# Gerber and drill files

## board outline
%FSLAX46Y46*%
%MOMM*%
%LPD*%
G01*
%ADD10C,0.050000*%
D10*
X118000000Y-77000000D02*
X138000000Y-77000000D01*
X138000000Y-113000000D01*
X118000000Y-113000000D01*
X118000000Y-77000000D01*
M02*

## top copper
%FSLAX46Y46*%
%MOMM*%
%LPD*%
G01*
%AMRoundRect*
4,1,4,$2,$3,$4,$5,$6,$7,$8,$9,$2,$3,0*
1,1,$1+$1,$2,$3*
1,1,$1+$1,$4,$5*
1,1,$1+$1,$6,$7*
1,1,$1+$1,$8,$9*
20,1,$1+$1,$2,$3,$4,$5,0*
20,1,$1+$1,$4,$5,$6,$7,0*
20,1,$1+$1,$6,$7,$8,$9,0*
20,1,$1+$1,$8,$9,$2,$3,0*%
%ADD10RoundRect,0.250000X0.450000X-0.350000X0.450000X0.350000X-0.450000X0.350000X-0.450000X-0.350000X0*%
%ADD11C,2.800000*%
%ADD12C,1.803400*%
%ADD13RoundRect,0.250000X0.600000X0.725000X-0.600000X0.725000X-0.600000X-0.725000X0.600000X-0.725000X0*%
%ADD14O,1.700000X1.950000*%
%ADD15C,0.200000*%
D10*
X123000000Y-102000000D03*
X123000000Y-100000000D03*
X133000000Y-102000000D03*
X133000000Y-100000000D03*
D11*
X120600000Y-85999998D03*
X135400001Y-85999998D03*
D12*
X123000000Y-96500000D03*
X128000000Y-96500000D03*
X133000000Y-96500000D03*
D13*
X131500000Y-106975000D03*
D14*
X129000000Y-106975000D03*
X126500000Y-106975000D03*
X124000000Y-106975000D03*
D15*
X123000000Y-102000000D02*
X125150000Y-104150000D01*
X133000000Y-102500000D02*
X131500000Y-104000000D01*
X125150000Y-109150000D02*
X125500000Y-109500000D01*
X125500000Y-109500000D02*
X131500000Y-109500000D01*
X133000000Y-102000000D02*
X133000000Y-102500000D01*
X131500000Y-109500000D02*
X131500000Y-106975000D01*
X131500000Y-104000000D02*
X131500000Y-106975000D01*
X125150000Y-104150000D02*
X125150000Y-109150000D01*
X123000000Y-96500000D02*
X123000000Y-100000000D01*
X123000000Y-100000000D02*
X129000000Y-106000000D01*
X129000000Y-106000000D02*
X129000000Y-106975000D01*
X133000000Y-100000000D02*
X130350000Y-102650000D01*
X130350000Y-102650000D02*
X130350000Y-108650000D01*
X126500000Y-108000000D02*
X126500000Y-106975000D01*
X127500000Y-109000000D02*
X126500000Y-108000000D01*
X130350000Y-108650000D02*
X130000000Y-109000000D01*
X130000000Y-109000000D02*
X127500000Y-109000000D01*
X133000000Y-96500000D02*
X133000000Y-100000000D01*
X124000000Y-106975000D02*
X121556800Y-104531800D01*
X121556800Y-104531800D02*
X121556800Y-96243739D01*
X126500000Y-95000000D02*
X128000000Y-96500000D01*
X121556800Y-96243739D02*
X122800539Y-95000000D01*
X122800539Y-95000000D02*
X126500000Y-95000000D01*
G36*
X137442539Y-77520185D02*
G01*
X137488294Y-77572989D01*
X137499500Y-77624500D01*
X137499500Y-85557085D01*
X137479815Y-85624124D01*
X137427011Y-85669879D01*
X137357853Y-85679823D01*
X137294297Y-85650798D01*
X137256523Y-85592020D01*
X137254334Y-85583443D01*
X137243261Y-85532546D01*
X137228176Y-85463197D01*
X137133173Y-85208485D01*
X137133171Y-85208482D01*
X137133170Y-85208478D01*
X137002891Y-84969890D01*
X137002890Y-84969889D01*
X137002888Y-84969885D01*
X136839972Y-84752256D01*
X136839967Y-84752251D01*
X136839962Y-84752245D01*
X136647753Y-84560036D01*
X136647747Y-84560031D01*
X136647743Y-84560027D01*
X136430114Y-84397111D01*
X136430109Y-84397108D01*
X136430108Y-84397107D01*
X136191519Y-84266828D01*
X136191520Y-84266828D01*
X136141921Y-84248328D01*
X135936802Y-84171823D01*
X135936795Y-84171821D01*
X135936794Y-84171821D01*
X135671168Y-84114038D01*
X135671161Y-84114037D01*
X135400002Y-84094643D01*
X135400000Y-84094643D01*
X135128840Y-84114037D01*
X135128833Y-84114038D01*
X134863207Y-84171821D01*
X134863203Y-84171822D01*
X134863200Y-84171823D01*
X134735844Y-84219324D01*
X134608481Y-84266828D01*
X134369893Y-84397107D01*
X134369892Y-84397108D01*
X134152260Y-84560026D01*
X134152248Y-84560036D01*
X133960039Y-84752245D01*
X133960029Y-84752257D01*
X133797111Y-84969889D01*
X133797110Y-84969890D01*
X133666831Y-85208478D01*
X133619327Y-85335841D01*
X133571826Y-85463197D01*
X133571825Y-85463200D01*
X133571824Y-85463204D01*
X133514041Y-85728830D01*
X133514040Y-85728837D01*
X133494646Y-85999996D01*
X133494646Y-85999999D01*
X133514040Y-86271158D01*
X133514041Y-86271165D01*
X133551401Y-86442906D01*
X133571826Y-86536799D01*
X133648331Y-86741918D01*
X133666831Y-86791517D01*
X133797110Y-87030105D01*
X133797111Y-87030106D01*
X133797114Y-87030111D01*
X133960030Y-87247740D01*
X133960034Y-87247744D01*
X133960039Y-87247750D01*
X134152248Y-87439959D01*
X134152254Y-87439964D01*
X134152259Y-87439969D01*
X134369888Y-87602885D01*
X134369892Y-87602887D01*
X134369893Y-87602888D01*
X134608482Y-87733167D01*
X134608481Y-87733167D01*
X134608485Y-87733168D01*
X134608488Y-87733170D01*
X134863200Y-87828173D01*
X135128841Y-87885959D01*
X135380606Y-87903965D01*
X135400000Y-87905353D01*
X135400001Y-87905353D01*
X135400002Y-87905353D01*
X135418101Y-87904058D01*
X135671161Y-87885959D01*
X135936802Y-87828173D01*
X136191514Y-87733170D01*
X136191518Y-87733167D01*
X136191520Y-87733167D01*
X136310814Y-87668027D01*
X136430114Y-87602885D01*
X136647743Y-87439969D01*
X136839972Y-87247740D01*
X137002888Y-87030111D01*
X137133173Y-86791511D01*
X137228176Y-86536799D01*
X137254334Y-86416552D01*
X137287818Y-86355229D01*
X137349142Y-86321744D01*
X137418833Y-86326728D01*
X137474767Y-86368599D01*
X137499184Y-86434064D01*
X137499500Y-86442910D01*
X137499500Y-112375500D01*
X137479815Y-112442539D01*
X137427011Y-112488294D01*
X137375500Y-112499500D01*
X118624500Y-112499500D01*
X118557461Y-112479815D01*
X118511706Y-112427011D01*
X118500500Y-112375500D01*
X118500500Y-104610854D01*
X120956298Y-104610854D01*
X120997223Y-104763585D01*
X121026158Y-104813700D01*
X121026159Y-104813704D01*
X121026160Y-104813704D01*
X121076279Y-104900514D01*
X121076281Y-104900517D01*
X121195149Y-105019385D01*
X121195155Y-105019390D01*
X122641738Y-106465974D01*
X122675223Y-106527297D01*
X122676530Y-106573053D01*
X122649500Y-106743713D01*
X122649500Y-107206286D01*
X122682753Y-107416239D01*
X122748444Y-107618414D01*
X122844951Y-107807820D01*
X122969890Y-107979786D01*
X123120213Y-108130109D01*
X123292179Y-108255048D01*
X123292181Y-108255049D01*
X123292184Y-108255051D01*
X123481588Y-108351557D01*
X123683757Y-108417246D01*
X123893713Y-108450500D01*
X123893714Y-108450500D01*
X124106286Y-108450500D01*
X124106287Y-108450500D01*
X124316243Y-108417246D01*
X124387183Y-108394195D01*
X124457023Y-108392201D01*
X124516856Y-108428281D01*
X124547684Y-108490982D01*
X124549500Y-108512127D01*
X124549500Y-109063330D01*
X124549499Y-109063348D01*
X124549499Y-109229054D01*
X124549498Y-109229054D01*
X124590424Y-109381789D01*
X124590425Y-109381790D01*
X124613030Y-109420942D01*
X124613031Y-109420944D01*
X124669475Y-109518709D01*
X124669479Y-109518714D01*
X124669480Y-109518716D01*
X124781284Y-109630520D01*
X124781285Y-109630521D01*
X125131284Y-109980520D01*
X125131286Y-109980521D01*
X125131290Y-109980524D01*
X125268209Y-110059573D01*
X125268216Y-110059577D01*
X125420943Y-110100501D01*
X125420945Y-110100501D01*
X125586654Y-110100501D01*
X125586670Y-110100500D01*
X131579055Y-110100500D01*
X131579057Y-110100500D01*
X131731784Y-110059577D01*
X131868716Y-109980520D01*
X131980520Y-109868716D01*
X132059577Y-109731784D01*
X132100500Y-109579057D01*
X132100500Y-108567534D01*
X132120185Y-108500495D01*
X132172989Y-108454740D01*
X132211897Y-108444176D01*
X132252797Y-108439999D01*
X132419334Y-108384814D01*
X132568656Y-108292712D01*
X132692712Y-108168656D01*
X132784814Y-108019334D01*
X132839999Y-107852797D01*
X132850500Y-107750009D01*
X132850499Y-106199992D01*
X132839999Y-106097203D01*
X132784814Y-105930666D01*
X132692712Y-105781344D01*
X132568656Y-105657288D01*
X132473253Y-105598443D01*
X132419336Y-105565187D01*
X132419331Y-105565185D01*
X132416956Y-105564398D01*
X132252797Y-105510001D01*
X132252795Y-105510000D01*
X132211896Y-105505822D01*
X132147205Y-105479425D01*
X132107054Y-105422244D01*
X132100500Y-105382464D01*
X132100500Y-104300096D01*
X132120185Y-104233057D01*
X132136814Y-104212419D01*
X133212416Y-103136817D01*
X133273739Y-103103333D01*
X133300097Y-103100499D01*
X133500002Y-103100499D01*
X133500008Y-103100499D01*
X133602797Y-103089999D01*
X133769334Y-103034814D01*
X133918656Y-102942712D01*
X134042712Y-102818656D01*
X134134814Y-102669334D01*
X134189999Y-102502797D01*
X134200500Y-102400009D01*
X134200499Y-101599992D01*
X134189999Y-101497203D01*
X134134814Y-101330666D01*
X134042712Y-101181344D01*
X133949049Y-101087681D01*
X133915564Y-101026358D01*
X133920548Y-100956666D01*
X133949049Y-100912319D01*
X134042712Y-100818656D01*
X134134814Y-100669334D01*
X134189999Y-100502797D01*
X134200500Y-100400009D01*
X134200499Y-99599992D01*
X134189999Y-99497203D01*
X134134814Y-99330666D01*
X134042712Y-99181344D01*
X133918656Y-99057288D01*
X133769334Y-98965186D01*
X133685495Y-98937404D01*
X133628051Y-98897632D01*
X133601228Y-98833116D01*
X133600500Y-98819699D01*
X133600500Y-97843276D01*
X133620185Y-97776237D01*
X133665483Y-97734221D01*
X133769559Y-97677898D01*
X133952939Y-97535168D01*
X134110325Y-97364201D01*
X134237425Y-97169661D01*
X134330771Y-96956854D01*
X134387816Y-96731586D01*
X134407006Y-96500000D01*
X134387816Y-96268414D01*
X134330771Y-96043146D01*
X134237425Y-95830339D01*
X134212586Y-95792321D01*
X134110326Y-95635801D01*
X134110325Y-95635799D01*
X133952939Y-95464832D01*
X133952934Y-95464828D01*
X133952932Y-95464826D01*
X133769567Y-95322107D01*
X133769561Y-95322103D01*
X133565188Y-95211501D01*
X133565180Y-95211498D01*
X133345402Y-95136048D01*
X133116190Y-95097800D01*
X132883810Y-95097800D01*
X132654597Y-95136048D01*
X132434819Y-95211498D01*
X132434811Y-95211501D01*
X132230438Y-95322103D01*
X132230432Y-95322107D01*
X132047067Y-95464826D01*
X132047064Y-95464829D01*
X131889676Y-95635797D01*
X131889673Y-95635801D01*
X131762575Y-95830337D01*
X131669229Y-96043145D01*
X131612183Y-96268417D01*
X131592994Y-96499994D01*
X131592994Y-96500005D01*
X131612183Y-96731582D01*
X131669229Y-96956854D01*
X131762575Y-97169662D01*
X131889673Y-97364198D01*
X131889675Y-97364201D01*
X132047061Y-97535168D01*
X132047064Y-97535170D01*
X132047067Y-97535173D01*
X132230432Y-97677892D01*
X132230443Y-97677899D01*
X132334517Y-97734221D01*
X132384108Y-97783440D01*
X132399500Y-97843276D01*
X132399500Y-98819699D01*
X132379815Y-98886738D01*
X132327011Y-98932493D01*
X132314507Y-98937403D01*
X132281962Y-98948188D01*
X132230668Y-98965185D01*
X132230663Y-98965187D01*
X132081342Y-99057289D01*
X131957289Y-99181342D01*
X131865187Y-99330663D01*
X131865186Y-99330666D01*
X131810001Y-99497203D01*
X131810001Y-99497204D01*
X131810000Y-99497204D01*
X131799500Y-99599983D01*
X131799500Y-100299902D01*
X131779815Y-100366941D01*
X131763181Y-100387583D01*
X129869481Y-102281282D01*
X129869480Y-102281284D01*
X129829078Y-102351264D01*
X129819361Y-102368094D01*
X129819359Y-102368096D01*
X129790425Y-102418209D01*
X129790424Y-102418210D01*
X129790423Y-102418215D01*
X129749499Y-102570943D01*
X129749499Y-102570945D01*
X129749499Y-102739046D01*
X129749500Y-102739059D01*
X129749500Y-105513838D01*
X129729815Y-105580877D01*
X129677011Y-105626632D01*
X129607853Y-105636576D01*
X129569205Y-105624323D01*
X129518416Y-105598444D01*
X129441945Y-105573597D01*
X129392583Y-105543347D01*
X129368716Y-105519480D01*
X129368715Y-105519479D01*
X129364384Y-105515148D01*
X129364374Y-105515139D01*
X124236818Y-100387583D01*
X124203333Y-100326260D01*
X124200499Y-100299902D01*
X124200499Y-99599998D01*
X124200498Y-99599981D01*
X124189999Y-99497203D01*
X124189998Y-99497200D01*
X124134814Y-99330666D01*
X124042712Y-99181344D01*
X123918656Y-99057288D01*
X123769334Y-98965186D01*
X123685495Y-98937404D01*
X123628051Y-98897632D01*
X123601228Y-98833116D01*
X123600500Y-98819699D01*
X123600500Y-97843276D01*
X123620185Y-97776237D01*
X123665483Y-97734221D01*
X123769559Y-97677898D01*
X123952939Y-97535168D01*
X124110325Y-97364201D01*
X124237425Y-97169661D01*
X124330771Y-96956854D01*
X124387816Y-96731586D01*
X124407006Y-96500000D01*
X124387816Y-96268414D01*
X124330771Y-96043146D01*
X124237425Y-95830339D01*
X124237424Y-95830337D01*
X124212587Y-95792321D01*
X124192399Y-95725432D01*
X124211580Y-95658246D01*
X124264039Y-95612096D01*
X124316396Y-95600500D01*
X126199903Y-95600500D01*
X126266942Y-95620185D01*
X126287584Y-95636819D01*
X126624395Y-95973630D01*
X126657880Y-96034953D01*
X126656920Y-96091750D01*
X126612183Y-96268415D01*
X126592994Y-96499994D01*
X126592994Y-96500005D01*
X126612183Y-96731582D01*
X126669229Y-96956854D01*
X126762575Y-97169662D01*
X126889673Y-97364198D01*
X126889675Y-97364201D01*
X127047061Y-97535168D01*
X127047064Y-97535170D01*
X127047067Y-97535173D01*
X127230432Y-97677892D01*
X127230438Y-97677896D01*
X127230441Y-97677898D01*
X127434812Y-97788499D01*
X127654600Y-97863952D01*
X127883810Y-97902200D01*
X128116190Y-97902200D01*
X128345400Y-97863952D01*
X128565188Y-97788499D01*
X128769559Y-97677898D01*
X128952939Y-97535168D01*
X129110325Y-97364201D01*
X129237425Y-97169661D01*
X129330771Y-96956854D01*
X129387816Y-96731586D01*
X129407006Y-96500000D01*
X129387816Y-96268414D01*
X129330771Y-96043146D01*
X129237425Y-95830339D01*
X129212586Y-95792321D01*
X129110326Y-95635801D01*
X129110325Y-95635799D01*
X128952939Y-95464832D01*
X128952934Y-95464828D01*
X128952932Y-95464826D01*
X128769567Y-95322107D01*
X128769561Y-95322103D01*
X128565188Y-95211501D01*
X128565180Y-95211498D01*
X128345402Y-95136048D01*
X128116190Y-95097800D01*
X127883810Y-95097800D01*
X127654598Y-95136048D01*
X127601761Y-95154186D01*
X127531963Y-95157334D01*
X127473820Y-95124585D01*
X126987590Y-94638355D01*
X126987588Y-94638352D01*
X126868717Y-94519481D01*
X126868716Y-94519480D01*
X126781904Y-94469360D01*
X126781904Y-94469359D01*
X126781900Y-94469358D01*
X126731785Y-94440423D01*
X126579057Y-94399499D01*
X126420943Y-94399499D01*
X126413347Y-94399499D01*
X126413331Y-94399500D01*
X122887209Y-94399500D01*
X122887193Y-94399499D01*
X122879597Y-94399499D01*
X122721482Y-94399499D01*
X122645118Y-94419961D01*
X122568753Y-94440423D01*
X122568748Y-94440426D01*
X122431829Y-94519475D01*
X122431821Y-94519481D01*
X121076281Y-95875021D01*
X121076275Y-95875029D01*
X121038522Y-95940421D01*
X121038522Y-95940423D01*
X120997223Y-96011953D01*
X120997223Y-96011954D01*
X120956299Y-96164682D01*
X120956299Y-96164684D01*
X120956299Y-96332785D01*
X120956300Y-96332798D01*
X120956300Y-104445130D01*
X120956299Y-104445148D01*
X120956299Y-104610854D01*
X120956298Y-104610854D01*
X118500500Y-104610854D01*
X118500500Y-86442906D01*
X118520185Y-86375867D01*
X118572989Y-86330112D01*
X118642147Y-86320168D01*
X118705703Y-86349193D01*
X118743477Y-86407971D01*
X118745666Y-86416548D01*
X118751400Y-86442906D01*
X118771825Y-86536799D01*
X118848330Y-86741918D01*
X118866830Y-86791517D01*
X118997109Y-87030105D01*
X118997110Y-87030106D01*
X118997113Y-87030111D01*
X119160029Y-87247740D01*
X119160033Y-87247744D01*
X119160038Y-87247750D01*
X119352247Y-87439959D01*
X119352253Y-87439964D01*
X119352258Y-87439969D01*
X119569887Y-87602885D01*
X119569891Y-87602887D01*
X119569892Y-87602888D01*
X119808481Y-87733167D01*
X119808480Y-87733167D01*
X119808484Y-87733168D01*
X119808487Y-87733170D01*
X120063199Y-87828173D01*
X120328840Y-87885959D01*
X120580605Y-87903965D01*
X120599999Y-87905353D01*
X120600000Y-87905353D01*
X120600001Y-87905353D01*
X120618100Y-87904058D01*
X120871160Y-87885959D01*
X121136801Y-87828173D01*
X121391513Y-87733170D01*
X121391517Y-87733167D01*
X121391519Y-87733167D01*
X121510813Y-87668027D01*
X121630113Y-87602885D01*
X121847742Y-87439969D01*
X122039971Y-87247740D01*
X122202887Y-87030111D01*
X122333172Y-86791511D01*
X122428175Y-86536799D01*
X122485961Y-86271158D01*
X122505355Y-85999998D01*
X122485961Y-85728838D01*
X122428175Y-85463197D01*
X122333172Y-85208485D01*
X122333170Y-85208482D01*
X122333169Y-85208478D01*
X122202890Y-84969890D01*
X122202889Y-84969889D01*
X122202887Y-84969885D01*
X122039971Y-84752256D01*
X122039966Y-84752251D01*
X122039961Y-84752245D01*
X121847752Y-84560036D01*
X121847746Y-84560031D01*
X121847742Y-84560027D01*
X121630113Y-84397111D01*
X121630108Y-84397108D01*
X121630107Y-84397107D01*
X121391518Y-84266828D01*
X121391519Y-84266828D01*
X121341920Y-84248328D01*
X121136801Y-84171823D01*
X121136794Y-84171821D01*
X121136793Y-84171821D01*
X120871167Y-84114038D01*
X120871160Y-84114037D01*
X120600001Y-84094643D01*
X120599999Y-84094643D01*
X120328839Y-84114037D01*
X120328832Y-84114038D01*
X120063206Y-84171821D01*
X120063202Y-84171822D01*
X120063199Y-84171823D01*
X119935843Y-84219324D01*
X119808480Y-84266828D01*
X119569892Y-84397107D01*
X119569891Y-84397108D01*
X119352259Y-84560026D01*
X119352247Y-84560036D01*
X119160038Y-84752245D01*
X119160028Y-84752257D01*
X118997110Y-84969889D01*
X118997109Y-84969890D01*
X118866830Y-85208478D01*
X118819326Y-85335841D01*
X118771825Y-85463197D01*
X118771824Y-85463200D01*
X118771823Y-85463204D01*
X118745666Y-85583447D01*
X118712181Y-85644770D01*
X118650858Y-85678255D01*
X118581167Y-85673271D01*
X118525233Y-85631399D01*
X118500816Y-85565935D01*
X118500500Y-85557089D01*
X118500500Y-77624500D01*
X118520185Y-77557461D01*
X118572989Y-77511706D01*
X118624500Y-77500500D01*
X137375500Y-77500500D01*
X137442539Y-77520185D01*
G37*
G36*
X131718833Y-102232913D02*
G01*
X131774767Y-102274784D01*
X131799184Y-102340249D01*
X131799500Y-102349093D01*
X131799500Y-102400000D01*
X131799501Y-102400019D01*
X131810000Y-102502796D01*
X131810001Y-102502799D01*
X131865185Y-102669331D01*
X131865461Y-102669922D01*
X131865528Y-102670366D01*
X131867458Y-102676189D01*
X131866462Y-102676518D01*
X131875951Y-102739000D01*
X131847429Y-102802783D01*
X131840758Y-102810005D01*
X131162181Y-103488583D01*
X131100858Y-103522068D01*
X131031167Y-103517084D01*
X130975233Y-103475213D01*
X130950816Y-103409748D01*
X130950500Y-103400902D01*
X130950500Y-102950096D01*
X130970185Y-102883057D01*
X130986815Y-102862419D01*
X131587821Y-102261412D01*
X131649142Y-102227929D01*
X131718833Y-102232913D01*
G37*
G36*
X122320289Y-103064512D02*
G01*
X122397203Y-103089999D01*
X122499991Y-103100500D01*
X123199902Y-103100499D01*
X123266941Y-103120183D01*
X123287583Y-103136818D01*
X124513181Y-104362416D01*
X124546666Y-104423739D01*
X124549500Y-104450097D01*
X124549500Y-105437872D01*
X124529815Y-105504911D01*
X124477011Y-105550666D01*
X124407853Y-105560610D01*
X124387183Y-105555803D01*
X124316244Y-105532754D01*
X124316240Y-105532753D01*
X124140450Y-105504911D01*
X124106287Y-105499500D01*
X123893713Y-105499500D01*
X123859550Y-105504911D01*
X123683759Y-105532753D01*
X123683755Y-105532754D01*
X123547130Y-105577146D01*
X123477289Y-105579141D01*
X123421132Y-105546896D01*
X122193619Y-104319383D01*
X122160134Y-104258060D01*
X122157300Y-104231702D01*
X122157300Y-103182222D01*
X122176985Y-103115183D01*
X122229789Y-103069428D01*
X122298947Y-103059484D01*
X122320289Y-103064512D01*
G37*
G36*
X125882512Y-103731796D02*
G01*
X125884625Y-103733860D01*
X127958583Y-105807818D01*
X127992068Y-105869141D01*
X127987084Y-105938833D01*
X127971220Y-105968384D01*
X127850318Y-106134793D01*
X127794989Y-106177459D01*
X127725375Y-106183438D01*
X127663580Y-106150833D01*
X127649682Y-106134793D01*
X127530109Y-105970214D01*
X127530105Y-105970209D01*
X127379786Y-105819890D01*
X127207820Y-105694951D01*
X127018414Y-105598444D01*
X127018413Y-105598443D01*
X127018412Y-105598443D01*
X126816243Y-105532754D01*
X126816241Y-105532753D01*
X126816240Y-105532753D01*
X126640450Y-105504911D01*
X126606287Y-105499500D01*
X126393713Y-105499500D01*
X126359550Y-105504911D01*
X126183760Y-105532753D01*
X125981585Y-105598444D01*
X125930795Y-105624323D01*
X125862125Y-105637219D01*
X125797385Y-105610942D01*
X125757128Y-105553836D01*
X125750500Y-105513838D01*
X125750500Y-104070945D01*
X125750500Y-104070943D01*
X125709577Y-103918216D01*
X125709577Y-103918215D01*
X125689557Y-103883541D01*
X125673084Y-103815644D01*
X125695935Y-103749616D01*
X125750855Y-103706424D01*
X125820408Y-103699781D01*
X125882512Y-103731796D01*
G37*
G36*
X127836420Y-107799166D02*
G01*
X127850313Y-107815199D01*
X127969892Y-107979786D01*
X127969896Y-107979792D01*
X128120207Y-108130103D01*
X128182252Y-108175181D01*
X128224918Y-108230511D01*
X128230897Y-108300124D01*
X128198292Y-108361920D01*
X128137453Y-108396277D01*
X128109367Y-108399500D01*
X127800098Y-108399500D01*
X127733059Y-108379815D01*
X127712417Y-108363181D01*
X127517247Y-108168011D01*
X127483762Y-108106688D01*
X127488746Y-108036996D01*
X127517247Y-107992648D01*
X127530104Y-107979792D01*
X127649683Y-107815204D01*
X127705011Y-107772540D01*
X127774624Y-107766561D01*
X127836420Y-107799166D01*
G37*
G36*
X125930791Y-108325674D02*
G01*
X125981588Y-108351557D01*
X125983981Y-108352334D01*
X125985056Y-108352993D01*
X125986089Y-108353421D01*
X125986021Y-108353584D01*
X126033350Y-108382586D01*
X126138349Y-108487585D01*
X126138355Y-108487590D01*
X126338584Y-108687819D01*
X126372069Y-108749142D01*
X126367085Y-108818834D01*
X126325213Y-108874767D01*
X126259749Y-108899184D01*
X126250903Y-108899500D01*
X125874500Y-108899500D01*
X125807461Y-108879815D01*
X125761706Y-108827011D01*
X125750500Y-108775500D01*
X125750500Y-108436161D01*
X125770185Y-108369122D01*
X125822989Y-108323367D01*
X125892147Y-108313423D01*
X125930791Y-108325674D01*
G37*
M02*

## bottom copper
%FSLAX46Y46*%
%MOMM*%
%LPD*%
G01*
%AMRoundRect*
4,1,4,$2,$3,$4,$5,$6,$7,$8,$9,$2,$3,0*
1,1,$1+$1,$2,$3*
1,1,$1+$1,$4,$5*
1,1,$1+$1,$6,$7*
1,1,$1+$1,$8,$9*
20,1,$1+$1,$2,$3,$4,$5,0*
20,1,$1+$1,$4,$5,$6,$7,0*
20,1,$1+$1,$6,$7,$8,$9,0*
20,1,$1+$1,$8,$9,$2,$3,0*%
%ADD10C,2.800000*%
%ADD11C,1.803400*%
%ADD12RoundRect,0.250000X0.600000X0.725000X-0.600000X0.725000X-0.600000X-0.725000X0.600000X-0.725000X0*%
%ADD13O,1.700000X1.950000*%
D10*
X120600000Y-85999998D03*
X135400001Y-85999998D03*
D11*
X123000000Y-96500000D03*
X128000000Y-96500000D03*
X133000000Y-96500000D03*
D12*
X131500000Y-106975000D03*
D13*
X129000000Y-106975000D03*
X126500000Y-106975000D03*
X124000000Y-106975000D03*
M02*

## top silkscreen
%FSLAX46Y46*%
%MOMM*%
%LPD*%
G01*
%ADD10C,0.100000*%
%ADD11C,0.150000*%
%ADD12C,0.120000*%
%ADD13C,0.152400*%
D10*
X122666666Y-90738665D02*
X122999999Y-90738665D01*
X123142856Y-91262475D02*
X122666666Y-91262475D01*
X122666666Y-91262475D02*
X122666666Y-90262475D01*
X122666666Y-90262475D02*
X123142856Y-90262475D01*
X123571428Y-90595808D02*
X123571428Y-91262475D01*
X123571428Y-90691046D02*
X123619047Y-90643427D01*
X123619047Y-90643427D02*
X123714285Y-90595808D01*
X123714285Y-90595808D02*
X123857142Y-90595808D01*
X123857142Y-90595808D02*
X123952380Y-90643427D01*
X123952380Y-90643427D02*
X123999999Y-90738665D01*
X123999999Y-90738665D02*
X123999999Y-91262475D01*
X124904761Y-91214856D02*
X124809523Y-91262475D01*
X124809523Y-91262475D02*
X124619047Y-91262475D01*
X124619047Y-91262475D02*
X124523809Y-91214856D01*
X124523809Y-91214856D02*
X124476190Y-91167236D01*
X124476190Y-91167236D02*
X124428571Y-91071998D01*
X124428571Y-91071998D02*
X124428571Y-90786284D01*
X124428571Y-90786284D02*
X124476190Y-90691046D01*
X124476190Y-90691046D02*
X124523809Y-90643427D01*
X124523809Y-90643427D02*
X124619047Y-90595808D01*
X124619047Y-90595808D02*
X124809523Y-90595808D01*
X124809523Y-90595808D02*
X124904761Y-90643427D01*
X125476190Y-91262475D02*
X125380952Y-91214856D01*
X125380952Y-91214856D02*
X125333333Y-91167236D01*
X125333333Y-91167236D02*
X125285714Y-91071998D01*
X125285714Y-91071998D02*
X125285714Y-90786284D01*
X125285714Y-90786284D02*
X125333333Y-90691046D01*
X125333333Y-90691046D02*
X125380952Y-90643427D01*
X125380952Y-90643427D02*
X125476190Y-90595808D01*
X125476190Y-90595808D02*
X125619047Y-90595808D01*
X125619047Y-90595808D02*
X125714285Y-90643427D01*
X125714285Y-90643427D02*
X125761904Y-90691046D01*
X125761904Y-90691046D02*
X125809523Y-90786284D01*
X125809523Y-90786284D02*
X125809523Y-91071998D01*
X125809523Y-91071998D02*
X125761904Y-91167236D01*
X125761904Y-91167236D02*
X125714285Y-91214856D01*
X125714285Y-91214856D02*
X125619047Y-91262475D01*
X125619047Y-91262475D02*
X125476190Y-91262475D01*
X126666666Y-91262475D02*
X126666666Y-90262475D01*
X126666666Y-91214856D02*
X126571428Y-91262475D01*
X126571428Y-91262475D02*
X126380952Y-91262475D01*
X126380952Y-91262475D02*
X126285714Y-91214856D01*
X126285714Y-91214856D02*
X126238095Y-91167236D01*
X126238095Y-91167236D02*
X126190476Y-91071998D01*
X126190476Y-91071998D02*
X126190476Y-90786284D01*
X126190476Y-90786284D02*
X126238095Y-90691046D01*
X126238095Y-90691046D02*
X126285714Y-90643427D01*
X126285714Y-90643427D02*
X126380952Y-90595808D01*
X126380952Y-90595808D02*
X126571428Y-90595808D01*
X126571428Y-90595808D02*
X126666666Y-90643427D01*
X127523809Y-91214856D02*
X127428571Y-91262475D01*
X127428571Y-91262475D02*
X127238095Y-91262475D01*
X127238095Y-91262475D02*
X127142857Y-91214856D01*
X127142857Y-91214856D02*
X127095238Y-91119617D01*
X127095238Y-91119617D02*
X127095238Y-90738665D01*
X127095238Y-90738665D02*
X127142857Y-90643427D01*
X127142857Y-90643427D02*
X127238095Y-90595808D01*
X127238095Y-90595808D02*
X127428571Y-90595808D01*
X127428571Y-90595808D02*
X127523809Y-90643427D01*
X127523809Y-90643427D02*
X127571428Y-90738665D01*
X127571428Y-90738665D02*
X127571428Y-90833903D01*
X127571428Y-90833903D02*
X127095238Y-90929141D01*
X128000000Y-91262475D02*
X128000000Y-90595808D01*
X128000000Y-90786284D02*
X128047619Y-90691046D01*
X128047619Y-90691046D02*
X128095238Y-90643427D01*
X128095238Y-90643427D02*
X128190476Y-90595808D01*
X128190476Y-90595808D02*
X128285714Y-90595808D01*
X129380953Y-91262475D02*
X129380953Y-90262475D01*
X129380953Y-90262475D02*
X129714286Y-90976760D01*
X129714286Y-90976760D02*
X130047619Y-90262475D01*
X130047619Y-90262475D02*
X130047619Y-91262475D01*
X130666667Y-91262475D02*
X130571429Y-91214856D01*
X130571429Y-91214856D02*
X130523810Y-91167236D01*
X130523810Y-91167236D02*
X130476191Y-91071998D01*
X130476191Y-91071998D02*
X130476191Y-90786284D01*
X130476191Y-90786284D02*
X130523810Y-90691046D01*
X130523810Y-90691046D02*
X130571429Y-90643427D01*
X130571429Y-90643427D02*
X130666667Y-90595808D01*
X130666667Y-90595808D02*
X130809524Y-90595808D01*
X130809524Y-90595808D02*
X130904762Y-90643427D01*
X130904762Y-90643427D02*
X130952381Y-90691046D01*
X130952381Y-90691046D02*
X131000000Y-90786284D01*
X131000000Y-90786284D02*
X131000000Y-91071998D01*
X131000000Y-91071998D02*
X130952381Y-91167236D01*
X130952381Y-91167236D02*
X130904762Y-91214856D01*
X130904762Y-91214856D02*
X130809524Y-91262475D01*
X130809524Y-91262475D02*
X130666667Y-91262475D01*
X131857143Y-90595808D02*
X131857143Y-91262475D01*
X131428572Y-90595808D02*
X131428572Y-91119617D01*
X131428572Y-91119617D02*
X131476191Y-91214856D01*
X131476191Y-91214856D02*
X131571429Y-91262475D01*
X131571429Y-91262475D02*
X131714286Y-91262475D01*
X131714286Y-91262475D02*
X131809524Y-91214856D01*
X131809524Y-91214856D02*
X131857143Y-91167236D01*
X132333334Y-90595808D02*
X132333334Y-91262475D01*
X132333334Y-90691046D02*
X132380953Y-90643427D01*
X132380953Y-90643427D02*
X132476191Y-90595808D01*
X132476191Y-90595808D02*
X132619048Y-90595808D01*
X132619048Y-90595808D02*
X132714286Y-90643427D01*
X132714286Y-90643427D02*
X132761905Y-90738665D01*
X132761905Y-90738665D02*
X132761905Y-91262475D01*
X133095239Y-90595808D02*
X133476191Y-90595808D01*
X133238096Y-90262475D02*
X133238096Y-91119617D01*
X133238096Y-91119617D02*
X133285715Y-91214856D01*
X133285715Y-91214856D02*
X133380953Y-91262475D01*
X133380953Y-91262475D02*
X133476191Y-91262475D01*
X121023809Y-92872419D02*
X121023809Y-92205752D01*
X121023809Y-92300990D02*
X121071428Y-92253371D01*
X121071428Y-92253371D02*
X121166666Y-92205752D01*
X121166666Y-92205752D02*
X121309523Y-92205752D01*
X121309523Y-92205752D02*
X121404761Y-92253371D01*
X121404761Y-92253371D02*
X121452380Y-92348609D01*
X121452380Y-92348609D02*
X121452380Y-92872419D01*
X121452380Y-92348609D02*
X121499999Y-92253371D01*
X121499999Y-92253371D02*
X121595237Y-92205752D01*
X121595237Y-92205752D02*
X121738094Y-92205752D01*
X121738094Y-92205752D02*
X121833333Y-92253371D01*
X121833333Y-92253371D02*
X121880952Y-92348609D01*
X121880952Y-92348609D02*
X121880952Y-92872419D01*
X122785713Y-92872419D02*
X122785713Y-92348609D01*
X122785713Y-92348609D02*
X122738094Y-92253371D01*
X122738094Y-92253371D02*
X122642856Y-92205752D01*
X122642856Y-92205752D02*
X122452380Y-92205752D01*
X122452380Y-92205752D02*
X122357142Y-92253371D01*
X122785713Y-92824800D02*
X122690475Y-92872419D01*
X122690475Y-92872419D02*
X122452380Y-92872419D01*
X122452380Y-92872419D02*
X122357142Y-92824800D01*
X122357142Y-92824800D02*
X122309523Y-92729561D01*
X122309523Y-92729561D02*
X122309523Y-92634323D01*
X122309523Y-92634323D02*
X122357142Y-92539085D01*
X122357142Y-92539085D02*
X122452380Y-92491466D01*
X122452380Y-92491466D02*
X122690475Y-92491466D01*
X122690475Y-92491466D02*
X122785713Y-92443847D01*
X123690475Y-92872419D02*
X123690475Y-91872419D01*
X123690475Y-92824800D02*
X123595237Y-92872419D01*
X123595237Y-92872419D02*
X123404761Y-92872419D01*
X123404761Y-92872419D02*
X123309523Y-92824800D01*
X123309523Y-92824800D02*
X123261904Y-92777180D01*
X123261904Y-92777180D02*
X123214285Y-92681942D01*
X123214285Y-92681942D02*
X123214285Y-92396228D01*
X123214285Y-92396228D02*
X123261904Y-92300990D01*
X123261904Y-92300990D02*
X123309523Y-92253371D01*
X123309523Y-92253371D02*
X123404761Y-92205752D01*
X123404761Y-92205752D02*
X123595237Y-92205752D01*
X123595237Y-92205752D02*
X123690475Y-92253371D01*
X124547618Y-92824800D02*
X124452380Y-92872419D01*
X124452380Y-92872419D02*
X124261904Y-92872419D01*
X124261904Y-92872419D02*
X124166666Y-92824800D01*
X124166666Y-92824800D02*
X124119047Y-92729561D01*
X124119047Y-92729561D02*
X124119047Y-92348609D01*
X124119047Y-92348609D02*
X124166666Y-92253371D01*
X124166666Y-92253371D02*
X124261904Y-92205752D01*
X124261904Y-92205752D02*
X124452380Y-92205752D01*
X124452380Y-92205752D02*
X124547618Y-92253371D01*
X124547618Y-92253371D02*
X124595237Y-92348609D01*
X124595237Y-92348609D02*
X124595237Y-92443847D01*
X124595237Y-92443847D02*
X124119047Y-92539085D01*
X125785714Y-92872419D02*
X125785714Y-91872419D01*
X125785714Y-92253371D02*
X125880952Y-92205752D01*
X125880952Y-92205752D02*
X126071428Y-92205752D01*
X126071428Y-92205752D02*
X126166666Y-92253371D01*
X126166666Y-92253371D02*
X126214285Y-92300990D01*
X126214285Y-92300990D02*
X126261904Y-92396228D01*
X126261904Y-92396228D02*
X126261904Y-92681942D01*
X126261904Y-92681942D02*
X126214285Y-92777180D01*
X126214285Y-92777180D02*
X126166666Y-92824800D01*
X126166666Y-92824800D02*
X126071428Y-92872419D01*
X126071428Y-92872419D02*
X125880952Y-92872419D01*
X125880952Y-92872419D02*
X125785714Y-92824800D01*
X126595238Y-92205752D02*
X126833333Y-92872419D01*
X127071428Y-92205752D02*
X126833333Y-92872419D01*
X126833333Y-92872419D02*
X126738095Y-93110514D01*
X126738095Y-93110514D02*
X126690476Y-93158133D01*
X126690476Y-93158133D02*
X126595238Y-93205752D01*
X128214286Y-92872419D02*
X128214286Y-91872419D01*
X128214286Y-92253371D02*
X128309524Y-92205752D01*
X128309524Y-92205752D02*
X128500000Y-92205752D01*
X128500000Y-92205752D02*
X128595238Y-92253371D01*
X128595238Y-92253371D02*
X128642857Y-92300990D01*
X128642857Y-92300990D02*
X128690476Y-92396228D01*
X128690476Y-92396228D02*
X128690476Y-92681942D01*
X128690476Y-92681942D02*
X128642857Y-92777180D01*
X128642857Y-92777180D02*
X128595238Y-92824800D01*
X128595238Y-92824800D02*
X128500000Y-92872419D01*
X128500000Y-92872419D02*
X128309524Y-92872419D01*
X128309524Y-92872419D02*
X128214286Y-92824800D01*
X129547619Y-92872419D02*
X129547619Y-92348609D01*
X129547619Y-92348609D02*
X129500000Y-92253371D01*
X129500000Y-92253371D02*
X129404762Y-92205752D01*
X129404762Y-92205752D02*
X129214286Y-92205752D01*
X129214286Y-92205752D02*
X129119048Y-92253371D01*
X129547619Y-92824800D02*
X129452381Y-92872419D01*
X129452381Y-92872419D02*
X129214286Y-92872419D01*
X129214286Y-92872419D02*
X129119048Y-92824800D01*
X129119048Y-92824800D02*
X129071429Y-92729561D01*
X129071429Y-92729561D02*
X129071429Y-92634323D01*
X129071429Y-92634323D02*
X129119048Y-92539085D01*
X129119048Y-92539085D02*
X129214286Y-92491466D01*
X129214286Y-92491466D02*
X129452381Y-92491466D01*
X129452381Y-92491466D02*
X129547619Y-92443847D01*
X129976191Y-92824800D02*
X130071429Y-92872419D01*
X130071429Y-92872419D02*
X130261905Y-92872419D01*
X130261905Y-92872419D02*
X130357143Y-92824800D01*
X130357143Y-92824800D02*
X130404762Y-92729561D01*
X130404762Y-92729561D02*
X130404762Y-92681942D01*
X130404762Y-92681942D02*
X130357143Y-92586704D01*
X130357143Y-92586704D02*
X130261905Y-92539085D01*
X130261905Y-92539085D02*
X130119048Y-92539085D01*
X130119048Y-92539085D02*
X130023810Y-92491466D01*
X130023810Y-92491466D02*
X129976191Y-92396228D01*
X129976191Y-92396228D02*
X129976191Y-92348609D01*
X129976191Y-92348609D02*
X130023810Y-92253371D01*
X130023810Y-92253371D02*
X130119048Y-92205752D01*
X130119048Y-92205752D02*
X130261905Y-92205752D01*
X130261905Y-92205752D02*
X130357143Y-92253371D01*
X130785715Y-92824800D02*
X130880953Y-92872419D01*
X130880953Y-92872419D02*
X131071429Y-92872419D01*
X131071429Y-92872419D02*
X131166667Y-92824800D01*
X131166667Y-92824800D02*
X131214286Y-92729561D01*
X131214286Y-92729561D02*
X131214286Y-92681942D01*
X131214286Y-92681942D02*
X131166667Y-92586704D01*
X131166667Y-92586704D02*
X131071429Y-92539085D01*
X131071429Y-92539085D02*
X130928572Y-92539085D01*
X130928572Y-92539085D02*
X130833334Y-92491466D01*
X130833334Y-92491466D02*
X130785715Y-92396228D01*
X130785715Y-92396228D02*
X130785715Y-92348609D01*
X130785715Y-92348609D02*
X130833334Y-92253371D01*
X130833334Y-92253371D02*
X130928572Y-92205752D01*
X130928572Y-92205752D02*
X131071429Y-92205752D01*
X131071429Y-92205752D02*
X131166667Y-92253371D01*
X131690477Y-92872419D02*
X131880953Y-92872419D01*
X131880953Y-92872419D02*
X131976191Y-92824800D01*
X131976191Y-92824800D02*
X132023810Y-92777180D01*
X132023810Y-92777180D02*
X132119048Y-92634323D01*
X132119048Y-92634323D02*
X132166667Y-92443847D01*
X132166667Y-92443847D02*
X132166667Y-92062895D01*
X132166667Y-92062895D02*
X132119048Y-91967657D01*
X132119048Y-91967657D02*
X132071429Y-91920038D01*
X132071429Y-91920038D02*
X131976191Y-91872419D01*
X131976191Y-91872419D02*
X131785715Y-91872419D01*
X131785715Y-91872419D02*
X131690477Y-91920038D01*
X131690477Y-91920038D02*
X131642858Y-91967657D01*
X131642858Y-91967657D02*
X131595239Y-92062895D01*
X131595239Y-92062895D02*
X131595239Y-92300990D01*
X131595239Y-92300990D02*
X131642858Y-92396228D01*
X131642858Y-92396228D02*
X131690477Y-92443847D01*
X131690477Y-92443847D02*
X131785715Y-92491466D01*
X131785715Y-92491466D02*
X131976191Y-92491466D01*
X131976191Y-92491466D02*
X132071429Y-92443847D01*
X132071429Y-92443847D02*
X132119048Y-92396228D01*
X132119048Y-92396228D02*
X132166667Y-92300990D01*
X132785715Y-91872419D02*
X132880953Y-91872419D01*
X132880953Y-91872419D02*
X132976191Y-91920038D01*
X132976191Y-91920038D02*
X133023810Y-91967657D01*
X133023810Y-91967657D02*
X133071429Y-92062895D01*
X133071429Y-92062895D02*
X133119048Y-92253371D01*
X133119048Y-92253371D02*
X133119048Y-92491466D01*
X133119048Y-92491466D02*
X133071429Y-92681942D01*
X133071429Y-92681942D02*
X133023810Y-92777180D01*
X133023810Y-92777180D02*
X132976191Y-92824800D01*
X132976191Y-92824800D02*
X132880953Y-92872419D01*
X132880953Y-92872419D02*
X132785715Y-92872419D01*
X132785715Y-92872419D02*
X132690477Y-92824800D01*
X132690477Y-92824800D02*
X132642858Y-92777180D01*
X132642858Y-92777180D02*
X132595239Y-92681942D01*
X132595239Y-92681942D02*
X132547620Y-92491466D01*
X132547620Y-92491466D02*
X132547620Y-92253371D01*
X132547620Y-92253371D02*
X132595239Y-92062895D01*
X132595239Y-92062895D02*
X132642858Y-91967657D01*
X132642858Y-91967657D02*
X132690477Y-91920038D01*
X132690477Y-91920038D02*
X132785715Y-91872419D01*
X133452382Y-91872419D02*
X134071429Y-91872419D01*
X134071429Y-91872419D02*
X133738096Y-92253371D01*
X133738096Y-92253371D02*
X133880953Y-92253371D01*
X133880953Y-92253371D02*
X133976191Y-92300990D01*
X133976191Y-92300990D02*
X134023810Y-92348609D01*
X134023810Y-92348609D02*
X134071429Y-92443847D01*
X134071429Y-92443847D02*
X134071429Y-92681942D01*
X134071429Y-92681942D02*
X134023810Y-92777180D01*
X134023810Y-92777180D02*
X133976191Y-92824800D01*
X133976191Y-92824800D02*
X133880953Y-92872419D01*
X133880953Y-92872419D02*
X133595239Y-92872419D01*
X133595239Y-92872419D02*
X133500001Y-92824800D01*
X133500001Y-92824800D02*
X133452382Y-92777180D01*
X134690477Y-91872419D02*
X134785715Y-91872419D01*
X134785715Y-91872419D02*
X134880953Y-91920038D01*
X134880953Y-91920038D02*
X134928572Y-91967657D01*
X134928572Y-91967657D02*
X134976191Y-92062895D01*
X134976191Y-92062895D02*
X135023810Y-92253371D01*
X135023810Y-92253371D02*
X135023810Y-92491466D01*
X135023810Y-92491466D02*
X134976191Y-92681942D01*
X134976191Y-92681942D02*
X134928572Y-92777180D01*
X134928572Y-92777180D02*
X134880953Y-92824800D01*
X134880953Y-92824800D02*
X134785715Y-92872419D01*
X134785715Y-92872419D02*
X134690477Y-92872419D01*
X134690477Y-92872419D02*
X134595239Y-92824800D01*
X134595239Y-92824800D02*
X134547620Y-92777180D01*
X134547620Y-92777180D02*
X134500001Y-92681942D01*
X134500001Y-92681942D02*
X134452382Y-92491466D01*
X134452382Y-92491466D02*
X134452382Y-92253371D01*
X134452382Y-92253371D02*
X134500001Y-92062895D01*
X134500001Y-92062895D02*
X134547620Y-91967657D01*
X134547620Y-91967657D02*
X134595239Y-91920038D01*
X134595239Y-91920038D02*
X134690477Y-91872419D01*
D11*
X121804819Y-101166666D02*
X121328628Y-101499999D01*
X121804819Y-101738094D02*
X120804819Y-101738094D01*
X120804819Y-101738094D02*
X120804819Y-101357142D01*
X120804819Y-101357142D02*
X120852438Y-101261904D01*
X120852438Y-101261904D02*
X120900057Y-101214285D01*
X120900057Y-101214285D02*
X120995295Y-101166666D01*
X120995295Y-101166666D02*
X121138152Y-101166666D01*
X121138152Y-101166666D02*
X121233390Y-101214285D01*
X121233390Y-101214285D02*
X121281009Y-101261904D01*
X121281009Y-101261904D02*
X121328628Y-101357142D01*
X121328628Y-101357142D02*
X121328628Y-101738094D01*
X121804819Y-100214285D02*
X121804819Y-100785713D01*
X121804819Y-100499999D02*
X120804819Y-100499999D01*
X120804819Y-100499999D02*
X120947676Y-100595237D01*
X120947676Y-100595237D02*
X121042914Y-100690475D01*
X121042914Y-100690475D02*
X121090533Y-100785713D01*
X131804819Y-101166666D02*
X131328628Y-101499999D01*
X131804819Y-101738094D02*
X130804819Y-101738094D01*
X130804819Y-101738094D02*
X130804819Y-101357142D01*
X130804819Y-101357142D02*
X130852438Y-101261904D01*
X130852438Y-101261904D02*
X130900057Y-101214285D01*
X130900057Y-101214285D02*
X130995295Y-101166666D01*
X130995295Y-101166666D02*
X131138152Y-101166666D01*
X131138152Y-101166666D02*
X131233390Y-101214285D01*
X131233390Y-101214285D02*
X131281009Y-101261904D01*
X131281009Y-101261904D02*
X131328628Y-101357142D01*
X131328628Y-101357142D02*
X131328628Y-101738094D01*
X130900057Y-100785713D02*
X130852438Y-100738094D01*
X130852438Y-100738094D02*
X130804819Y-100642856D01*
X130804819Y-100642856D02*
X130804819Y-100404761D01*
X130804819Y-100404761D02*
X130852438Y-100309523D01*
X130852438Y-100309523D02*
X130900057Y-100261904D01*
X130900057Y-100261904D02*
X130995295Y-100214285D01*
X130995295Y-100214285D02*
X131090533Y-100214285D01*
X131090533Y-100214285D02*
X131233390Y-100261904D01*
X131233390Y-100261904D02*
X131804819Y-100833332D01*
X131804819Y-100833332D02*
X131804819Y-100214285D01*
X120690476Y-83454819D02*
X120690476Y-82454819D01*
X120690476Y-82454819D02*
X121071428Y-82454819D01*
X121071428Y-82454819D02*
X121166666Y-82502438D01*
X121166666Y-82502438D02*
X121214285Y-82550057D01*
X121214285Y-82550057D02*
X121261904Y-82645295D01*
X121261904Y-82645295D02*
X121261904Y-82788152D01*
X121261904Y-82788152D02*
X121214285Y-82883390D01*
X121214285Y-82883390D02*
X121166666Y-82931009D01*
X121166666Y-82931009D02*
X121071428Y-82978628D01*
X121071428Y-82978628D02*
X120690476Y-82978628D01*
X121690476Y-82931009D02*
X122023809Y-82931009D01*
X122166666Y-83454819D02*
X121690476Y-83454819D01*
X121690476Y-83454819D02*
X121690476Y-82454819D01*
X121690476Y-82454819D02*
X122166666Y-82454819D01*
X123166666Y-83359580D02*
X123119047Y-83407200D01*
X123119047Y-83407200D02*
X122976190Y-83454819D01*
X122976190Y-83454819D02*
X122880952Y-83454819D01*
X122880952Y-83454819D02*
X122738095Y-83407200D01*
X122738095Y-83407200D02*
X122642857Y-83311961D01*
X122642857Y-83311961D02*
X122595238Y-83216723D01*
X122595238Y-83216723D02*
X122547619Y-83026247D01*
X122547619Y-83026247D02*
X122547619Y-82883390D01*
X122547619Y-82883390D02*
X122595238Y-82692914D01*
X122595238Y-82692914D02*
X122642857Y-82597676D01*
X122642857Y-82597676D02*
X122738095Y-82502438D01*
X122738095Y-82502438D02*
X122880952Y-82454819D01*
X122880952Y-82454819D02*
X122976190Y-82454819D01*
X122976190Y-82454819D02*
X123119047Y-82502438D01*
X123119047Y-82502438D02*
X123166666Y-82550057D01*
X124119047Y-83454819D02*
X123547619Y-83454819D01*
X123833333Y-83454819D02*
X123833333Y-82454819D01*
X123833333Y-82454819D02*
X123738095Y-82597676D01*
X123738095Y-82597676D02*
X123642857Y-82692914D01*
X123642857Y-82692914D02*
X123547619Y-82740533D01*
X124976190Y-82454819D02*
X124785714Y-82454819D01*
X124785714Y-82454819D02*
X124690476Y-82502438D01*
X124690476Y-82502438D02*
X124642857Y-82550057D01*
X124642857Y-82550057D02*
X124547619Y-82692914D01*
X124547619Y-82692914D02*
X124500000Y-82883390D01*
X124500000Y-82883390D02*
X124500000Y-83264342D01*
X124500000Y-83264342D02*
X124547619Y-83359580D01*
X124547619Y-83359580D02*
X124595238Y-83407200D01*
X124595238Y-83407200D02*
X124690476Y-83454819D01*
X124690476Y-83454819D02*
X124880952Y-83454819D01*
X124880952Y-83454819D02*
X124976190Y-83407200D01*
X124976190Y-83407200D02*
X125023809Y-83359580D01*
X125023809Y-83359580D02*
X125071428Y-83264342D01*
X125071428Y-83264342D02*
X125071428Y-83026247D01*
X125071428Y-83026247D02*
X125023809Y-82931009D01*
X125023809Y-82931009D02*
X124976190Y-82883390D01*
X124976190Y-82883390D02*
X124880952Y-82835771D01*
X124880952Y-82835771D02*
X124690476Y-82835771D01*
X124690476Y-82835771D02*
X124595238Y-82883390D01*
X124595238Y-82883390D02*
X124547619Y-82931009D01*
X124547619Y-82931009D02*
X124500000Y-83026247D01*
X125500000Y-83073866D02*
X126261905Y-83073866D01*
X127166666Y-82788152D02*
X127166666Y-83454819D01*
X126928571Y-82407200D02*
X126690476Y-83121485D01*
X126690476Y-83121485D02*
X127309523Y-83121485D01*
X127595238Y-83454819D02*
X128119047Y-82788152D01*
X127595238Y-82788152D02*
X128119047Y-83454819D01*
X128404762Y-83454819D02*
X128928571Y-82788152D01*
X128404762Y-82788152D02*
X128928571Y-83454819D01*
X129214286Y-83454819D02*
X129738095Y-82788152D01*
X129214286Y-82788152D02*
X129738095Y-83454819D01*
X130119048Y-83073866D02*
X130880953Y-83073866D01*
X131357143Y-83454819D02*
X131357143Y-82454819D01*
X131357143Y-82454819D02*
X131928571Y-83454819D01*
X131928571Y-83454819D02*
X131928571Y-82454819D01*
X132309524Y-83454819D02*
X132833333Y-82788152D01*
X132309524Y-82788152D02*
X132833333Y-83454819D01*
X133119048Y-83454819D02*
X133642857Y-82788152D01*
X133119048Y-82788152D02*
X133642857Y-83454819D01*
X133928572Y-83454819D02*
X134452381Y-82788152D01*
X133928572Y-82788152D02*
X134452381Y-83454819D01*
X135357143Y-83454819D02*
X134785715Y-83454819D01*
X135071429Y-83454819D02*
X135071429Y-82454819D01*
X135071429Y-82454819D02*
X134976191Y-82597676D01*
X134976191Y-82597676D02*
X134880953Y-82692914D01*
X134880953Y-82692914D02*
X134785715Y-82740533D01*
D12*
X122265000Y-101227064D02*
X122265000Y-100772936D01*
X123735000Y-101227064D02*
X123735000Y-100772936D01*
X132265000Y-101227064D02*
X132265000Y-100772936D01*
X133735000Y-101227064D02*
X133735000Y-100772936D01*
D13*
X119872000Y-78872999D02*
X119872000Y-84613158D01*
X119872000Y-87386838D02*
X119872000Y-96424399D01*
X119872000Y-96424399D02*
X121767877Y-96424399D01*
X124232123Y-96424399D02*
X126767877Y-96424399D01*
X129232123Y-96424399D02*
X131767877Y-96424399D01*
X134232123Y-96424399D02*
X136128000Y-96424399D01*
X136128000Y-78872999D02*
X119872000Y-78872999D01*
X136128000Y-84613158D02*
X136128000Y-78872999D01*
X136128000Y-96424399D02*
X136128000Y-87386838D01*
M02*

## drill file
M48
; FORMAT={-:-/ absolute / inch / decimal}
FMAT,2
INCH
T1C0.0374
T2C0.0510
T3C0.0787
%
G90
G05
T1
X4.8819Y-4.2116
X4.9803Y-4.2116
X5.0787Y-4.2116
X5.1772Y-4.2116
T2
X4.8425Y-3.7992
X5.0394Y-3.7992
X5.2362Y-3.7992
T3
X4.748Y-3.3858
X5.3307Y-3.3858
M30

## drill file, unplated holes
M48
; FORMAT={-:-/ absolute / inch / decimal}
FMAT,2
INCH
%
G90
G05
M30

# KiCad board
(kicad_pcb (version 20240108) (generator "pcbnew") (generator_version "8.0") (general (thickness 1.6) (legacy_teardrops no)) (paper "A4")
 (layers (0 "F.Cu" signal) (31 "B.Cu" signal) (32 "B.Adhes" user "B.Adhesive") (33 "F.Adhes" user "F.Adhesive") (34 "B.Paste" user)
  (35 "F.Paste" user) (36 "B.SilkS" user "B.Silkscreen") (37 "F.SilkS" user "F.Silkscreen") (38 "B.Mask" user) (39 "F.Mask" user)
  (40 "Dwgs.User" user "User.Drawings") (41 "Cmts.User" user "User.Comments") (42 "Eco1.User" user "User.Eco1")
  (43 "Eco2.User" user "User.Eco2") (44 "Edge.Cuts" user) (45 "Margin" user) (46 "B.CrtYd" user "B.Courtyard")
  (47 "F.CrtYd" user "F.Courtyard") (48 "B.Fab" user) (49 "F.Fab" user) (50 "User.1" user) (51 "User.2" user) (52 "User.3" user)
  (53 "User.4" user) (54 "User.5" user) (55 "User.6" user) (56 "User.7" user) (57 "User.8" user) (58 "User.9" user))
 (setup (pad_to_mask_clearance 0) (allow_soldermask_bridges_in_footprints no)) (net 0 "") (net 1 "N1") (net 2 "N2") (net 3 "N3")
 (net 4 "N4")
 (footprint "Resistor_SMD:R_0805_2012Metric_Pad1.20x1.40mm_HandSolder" (layer "F.Cu") (at 123 101 90)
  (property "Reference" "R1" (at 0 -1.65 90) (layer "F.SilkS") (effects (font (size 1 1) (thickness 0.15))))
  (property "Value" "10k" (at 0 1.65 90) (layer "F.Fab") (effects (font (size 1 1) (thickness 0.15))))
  (fp_line (start -0.227064 -0.735) (end 0.227064 -0.735) (stroke (width 0.12) (type solid)) (layer "F.SilkS"))
  (fp_line (start -0.227064 0.735) (end 0.227064 0.735) (stroke (width 0.12) (type solid)) (layer "F.SilkS"))
  (pad "1" smd roundrect (at -1 0 90) (size 1.2 1.4) (layers "F.Cu" "F.Paste" "F.Mask") (roundrect_rratio 0.208333) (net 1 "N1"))
  (pad "2" smd roundrect (at 1 0 90) (size 1.2 1.4) (layers "F.Cu" "F.Paste" "F.Mask") (roundrect_rratio 0.208333) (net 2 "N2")))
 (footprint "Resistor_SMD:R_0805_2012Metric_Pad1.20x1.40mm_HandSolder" (layer "F.Cu") (at 133 101 90)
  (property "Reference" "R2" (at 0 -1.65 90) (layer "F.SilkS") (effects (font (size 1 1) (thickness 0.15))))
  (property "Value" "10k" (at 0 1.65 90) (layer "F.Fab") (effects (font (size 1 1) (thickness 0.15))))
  (fp_line (start -0.227064 -0.735) (end 0.227064 -0.735) (stroke (width 0.12) (type solid)) (layer "F.SilkS"))
  (fp_line (start -0.227064 0.735) (end 0.227064 0.735) (stroke (width 0.12) (type solid)) (layer "F.SilkS"))
  (pad "1" smd roundrect (at -1 0 90) (size 1.2 1.4) (layers "F.Cu" "F.Paste" "F.Mask") (roundrect_rratio 0.208333) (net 1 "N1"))
  (pad "2" smd roundrect (at 1 0 90) (size 1.2 1.4) (layers "F.Cu" "F.Paste" "F.Mask") (roundrect_rratio 0.208333) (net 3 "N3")))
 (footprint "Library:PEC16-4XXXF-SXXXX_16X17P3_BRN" (layer "F.Cu") (at 135.400001 85.999998)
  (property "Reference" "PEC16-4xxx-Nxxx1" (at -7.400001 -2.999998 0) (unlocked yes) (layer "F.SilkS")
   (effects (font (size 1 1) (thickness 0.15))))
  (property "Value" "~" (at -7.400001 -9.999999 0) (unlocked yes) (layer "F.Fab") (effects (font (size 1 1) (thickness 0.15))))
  (fp_line (start -15.528001 -7.126999) (end -15.528001 -1.38684) (stroke (width 0.1524) (type solid)) (layer "F.SilkS"))
  (fp_line (start -15.528001 1.38684) (end -15.528001 10.424401) (stroke (width 0.1524) (type solid)) (layer "F.SilkS"))
  (fp_line (start -15.528001 10.424401) (end -13.632124 10.424401) (stroke (width 0.1524) (type solid)) (layer "F.SilkS"))
  (fp_line (start -11.167878 10.424401) (end -8.632124 10.424401) (stroke (width 0.1524) (type solid)) (layer "F.SilkS"))
  (fp_line (start -6.167878 10.424401) (end -3.632124 10.424401) (stroke (width 0.1524) (type solid)) (layer "F.SilkS"))
  (fp_line (start -1.167878 10.424401) (end 0.727999 10.424401) (stroke (width 0.1524) (type solid)) (layer "F.SilkS"))
  (fp_line (start 0.727999 -7.126999) (end -15.528001 -7.126999) (stroke (width 0.1524) (type solid)) (layer "F.SilkS"))
  (fp_line (start 0.727999 -1.38684) (end 0.727999 -7.126999) (stroke (width 0.1524) (type solid)) (layer "F.SilkS"))
  (fp_line (start 0.727999 10.424401) (end 0.727999 1.38684) (stroke (width 0.1524) (type solid)) (layer "F.SilkS"))
  (pad "" thru_hole circle (at -14.800001 0) (size 2.8 2.8) (drill 2) (layers "*.Cu" "*.Mask") (remove_unused_layers no))
  (pad "" thru_hole circle (at 0 0) (size 2.8 2.8) (drill 2) (layers "*.Cu" "*.Mask") (remove_unused_layers no))
  (pad "1" thru_hole circle (at -12.400001 10.500002) (size 1.8034 1.8034) (drill 1.2954) (layers "*.Cu" "*.Mask") (remove_unused_layers no)
   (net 2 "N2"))
  (pad "2" thru_hole circle (at -7.400001 10.500002) (size 1.8034 1.8034) (drill 1.2954) (layers "*.Cu" "*.Mask") (remove_unused_layers no)
   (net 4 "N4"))
  (pad "3" thru_hole circle (at -2.400001 10.500002) (size 1.8034 1.8034) (drill 1.2954) (layers "*.Cu" "*.Mask") (remove_unused_layers no)
   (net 3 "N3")))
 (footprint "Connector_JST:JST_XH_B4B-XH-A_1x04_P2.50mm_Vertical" (layer "B.Cu") (at 131.5 106.975 180)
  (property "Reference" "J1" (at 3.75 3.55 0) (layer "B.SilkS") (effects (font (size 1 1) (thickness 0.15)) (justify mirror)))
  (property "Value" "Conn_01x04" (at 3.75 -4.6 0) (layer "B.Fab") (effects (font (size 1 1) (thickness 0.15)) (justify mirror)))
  (pad "1" thru_hole roundrect (at 0 0 180) (size 1.7 1.95) (drill 0.95) (layers "*.Cu" "*.Mask") (remove_unused_layers no)
   (roundrect_rratio 0.147059) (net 1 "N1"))
  (pad "2" thru_hole oval (at 2.5 0 180) (size 1.7 1.95) (drill 0.95) (layers "*.Cu" "*.Mask") (remove_unused_layers no) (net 2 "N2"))
  (pad "3" thru_hole oval (at 5 0 180) (size 1.7 1.95) (drill 0.95) (layers "*.Cu" "*.Mask") (remove_unused_layers no) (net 3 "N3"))
  (pad "4" thru_hole oval (at 7.5 0 180) (size 1.7 1.95) (drill 0.95) (layers "*.Cu" "*.Mask") (remove_unused_layers no) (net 4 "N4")))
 (gr_rect (start 118 77) (end 138 113) (stroke (width 0.05) (type default)) (fill none) (layer "Edge.Cuts"))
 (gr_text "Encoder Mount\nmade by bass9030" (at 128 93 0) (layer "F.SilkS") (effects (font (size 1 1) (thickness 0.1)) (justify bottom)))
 (segment (start 123 102) (end 125.15 104.15) (width 0.2) (layer "F.Cu") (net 1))
 (segment (start 133 102.5) (end 131.5 104) (width 0.2) (layer "F.Cu") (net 1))
 (segment (start 125.15 109.15) (end 125.5 109.5) (width 0.2) (layer "F.Cu") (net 1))
 (segment (start 125.5 109.5) (end 131.5 109.5) (width 0.2) (layer "F.Cu") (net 1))
 (segment (start 133 102) (end 133 102.5) (width 0.2) (layer "F.Cu") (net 1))
 (segment (start 131.5 109.5) (end 131.5 106.975) (width 0.2) (layer "F.Cu") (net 1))
 (segment (start 131.5 104) (end 131.5 106.975) (width 0.2) (layer "F.Cu") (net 1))
 (segment (start 125.15 104.15) (end 125.15 109.15) (width 0.2) (layer "F.Cu") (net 1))
 (segment (start 123 96.5) (end 123 100) (width 0.2) (layer "F.Cu") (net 2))
 (segment (start 123 100) (end 129 106) (width 0.2) (layer "F.Cu") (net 2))
 (segment (start 129 106) (end 129 106.975) (width 0.2) (layer "F.Cu") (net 2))
 (segment (start 133 100) (end 130.35 102.65) (width 0.2) (layer "F.Cu") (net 3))
 (segment (start 130.35 102.65) (end 130.35 108.65) (width 0.2) (layer "F.Cu") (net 3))
 (segment (start 126.5 108) (end 126.5 106.975) (width 0.2) (layer "F.Cu") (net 3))
 (segment (start 127.5 109) (end 126.5 108) (width 0.2) (layer "F.Cu") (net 3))
 (segment (start 130.35 108.65) (end 130 109) (width 0.2) (layer "F.Cu") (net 3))
 (segment (start 130 109) (end 127.5 109) (width 0.2) (layer "F.Cu") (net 3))
 (segment (start 133 96.5) (end 133 100) (width 0.2) (layer "F.Cu") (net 3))
 (segment (start 124 106.975) (end 121.5568 104.5318) (width 0.2) (layer "F.Cu") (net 4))
 (segment (start 121.5568 104.5318) (end 121.5568 96.243739) (width 0.2) (layer "F.Cu") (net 4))
 (segment (start 126.5 95) (end 128 96.5) (width 0.2) (layer "F.Cu") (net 4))
 (segment (start 121.5568 96.243739) (end 122.800539 95) (width 0.2) (layer "F.Cu") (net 4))
 (segment (start 122.800539 95) (end 126.5 95) (width 0.2) (layer "F.Cu") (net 4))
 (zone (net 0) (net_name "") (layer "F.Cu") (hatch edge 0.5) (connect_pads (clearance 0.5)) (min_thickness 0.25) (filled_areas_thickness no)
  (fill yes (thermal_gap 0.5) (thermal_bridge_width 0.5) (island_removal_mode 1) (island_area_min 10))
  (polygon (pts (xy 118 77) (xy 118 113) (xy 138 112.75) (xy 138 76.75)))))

